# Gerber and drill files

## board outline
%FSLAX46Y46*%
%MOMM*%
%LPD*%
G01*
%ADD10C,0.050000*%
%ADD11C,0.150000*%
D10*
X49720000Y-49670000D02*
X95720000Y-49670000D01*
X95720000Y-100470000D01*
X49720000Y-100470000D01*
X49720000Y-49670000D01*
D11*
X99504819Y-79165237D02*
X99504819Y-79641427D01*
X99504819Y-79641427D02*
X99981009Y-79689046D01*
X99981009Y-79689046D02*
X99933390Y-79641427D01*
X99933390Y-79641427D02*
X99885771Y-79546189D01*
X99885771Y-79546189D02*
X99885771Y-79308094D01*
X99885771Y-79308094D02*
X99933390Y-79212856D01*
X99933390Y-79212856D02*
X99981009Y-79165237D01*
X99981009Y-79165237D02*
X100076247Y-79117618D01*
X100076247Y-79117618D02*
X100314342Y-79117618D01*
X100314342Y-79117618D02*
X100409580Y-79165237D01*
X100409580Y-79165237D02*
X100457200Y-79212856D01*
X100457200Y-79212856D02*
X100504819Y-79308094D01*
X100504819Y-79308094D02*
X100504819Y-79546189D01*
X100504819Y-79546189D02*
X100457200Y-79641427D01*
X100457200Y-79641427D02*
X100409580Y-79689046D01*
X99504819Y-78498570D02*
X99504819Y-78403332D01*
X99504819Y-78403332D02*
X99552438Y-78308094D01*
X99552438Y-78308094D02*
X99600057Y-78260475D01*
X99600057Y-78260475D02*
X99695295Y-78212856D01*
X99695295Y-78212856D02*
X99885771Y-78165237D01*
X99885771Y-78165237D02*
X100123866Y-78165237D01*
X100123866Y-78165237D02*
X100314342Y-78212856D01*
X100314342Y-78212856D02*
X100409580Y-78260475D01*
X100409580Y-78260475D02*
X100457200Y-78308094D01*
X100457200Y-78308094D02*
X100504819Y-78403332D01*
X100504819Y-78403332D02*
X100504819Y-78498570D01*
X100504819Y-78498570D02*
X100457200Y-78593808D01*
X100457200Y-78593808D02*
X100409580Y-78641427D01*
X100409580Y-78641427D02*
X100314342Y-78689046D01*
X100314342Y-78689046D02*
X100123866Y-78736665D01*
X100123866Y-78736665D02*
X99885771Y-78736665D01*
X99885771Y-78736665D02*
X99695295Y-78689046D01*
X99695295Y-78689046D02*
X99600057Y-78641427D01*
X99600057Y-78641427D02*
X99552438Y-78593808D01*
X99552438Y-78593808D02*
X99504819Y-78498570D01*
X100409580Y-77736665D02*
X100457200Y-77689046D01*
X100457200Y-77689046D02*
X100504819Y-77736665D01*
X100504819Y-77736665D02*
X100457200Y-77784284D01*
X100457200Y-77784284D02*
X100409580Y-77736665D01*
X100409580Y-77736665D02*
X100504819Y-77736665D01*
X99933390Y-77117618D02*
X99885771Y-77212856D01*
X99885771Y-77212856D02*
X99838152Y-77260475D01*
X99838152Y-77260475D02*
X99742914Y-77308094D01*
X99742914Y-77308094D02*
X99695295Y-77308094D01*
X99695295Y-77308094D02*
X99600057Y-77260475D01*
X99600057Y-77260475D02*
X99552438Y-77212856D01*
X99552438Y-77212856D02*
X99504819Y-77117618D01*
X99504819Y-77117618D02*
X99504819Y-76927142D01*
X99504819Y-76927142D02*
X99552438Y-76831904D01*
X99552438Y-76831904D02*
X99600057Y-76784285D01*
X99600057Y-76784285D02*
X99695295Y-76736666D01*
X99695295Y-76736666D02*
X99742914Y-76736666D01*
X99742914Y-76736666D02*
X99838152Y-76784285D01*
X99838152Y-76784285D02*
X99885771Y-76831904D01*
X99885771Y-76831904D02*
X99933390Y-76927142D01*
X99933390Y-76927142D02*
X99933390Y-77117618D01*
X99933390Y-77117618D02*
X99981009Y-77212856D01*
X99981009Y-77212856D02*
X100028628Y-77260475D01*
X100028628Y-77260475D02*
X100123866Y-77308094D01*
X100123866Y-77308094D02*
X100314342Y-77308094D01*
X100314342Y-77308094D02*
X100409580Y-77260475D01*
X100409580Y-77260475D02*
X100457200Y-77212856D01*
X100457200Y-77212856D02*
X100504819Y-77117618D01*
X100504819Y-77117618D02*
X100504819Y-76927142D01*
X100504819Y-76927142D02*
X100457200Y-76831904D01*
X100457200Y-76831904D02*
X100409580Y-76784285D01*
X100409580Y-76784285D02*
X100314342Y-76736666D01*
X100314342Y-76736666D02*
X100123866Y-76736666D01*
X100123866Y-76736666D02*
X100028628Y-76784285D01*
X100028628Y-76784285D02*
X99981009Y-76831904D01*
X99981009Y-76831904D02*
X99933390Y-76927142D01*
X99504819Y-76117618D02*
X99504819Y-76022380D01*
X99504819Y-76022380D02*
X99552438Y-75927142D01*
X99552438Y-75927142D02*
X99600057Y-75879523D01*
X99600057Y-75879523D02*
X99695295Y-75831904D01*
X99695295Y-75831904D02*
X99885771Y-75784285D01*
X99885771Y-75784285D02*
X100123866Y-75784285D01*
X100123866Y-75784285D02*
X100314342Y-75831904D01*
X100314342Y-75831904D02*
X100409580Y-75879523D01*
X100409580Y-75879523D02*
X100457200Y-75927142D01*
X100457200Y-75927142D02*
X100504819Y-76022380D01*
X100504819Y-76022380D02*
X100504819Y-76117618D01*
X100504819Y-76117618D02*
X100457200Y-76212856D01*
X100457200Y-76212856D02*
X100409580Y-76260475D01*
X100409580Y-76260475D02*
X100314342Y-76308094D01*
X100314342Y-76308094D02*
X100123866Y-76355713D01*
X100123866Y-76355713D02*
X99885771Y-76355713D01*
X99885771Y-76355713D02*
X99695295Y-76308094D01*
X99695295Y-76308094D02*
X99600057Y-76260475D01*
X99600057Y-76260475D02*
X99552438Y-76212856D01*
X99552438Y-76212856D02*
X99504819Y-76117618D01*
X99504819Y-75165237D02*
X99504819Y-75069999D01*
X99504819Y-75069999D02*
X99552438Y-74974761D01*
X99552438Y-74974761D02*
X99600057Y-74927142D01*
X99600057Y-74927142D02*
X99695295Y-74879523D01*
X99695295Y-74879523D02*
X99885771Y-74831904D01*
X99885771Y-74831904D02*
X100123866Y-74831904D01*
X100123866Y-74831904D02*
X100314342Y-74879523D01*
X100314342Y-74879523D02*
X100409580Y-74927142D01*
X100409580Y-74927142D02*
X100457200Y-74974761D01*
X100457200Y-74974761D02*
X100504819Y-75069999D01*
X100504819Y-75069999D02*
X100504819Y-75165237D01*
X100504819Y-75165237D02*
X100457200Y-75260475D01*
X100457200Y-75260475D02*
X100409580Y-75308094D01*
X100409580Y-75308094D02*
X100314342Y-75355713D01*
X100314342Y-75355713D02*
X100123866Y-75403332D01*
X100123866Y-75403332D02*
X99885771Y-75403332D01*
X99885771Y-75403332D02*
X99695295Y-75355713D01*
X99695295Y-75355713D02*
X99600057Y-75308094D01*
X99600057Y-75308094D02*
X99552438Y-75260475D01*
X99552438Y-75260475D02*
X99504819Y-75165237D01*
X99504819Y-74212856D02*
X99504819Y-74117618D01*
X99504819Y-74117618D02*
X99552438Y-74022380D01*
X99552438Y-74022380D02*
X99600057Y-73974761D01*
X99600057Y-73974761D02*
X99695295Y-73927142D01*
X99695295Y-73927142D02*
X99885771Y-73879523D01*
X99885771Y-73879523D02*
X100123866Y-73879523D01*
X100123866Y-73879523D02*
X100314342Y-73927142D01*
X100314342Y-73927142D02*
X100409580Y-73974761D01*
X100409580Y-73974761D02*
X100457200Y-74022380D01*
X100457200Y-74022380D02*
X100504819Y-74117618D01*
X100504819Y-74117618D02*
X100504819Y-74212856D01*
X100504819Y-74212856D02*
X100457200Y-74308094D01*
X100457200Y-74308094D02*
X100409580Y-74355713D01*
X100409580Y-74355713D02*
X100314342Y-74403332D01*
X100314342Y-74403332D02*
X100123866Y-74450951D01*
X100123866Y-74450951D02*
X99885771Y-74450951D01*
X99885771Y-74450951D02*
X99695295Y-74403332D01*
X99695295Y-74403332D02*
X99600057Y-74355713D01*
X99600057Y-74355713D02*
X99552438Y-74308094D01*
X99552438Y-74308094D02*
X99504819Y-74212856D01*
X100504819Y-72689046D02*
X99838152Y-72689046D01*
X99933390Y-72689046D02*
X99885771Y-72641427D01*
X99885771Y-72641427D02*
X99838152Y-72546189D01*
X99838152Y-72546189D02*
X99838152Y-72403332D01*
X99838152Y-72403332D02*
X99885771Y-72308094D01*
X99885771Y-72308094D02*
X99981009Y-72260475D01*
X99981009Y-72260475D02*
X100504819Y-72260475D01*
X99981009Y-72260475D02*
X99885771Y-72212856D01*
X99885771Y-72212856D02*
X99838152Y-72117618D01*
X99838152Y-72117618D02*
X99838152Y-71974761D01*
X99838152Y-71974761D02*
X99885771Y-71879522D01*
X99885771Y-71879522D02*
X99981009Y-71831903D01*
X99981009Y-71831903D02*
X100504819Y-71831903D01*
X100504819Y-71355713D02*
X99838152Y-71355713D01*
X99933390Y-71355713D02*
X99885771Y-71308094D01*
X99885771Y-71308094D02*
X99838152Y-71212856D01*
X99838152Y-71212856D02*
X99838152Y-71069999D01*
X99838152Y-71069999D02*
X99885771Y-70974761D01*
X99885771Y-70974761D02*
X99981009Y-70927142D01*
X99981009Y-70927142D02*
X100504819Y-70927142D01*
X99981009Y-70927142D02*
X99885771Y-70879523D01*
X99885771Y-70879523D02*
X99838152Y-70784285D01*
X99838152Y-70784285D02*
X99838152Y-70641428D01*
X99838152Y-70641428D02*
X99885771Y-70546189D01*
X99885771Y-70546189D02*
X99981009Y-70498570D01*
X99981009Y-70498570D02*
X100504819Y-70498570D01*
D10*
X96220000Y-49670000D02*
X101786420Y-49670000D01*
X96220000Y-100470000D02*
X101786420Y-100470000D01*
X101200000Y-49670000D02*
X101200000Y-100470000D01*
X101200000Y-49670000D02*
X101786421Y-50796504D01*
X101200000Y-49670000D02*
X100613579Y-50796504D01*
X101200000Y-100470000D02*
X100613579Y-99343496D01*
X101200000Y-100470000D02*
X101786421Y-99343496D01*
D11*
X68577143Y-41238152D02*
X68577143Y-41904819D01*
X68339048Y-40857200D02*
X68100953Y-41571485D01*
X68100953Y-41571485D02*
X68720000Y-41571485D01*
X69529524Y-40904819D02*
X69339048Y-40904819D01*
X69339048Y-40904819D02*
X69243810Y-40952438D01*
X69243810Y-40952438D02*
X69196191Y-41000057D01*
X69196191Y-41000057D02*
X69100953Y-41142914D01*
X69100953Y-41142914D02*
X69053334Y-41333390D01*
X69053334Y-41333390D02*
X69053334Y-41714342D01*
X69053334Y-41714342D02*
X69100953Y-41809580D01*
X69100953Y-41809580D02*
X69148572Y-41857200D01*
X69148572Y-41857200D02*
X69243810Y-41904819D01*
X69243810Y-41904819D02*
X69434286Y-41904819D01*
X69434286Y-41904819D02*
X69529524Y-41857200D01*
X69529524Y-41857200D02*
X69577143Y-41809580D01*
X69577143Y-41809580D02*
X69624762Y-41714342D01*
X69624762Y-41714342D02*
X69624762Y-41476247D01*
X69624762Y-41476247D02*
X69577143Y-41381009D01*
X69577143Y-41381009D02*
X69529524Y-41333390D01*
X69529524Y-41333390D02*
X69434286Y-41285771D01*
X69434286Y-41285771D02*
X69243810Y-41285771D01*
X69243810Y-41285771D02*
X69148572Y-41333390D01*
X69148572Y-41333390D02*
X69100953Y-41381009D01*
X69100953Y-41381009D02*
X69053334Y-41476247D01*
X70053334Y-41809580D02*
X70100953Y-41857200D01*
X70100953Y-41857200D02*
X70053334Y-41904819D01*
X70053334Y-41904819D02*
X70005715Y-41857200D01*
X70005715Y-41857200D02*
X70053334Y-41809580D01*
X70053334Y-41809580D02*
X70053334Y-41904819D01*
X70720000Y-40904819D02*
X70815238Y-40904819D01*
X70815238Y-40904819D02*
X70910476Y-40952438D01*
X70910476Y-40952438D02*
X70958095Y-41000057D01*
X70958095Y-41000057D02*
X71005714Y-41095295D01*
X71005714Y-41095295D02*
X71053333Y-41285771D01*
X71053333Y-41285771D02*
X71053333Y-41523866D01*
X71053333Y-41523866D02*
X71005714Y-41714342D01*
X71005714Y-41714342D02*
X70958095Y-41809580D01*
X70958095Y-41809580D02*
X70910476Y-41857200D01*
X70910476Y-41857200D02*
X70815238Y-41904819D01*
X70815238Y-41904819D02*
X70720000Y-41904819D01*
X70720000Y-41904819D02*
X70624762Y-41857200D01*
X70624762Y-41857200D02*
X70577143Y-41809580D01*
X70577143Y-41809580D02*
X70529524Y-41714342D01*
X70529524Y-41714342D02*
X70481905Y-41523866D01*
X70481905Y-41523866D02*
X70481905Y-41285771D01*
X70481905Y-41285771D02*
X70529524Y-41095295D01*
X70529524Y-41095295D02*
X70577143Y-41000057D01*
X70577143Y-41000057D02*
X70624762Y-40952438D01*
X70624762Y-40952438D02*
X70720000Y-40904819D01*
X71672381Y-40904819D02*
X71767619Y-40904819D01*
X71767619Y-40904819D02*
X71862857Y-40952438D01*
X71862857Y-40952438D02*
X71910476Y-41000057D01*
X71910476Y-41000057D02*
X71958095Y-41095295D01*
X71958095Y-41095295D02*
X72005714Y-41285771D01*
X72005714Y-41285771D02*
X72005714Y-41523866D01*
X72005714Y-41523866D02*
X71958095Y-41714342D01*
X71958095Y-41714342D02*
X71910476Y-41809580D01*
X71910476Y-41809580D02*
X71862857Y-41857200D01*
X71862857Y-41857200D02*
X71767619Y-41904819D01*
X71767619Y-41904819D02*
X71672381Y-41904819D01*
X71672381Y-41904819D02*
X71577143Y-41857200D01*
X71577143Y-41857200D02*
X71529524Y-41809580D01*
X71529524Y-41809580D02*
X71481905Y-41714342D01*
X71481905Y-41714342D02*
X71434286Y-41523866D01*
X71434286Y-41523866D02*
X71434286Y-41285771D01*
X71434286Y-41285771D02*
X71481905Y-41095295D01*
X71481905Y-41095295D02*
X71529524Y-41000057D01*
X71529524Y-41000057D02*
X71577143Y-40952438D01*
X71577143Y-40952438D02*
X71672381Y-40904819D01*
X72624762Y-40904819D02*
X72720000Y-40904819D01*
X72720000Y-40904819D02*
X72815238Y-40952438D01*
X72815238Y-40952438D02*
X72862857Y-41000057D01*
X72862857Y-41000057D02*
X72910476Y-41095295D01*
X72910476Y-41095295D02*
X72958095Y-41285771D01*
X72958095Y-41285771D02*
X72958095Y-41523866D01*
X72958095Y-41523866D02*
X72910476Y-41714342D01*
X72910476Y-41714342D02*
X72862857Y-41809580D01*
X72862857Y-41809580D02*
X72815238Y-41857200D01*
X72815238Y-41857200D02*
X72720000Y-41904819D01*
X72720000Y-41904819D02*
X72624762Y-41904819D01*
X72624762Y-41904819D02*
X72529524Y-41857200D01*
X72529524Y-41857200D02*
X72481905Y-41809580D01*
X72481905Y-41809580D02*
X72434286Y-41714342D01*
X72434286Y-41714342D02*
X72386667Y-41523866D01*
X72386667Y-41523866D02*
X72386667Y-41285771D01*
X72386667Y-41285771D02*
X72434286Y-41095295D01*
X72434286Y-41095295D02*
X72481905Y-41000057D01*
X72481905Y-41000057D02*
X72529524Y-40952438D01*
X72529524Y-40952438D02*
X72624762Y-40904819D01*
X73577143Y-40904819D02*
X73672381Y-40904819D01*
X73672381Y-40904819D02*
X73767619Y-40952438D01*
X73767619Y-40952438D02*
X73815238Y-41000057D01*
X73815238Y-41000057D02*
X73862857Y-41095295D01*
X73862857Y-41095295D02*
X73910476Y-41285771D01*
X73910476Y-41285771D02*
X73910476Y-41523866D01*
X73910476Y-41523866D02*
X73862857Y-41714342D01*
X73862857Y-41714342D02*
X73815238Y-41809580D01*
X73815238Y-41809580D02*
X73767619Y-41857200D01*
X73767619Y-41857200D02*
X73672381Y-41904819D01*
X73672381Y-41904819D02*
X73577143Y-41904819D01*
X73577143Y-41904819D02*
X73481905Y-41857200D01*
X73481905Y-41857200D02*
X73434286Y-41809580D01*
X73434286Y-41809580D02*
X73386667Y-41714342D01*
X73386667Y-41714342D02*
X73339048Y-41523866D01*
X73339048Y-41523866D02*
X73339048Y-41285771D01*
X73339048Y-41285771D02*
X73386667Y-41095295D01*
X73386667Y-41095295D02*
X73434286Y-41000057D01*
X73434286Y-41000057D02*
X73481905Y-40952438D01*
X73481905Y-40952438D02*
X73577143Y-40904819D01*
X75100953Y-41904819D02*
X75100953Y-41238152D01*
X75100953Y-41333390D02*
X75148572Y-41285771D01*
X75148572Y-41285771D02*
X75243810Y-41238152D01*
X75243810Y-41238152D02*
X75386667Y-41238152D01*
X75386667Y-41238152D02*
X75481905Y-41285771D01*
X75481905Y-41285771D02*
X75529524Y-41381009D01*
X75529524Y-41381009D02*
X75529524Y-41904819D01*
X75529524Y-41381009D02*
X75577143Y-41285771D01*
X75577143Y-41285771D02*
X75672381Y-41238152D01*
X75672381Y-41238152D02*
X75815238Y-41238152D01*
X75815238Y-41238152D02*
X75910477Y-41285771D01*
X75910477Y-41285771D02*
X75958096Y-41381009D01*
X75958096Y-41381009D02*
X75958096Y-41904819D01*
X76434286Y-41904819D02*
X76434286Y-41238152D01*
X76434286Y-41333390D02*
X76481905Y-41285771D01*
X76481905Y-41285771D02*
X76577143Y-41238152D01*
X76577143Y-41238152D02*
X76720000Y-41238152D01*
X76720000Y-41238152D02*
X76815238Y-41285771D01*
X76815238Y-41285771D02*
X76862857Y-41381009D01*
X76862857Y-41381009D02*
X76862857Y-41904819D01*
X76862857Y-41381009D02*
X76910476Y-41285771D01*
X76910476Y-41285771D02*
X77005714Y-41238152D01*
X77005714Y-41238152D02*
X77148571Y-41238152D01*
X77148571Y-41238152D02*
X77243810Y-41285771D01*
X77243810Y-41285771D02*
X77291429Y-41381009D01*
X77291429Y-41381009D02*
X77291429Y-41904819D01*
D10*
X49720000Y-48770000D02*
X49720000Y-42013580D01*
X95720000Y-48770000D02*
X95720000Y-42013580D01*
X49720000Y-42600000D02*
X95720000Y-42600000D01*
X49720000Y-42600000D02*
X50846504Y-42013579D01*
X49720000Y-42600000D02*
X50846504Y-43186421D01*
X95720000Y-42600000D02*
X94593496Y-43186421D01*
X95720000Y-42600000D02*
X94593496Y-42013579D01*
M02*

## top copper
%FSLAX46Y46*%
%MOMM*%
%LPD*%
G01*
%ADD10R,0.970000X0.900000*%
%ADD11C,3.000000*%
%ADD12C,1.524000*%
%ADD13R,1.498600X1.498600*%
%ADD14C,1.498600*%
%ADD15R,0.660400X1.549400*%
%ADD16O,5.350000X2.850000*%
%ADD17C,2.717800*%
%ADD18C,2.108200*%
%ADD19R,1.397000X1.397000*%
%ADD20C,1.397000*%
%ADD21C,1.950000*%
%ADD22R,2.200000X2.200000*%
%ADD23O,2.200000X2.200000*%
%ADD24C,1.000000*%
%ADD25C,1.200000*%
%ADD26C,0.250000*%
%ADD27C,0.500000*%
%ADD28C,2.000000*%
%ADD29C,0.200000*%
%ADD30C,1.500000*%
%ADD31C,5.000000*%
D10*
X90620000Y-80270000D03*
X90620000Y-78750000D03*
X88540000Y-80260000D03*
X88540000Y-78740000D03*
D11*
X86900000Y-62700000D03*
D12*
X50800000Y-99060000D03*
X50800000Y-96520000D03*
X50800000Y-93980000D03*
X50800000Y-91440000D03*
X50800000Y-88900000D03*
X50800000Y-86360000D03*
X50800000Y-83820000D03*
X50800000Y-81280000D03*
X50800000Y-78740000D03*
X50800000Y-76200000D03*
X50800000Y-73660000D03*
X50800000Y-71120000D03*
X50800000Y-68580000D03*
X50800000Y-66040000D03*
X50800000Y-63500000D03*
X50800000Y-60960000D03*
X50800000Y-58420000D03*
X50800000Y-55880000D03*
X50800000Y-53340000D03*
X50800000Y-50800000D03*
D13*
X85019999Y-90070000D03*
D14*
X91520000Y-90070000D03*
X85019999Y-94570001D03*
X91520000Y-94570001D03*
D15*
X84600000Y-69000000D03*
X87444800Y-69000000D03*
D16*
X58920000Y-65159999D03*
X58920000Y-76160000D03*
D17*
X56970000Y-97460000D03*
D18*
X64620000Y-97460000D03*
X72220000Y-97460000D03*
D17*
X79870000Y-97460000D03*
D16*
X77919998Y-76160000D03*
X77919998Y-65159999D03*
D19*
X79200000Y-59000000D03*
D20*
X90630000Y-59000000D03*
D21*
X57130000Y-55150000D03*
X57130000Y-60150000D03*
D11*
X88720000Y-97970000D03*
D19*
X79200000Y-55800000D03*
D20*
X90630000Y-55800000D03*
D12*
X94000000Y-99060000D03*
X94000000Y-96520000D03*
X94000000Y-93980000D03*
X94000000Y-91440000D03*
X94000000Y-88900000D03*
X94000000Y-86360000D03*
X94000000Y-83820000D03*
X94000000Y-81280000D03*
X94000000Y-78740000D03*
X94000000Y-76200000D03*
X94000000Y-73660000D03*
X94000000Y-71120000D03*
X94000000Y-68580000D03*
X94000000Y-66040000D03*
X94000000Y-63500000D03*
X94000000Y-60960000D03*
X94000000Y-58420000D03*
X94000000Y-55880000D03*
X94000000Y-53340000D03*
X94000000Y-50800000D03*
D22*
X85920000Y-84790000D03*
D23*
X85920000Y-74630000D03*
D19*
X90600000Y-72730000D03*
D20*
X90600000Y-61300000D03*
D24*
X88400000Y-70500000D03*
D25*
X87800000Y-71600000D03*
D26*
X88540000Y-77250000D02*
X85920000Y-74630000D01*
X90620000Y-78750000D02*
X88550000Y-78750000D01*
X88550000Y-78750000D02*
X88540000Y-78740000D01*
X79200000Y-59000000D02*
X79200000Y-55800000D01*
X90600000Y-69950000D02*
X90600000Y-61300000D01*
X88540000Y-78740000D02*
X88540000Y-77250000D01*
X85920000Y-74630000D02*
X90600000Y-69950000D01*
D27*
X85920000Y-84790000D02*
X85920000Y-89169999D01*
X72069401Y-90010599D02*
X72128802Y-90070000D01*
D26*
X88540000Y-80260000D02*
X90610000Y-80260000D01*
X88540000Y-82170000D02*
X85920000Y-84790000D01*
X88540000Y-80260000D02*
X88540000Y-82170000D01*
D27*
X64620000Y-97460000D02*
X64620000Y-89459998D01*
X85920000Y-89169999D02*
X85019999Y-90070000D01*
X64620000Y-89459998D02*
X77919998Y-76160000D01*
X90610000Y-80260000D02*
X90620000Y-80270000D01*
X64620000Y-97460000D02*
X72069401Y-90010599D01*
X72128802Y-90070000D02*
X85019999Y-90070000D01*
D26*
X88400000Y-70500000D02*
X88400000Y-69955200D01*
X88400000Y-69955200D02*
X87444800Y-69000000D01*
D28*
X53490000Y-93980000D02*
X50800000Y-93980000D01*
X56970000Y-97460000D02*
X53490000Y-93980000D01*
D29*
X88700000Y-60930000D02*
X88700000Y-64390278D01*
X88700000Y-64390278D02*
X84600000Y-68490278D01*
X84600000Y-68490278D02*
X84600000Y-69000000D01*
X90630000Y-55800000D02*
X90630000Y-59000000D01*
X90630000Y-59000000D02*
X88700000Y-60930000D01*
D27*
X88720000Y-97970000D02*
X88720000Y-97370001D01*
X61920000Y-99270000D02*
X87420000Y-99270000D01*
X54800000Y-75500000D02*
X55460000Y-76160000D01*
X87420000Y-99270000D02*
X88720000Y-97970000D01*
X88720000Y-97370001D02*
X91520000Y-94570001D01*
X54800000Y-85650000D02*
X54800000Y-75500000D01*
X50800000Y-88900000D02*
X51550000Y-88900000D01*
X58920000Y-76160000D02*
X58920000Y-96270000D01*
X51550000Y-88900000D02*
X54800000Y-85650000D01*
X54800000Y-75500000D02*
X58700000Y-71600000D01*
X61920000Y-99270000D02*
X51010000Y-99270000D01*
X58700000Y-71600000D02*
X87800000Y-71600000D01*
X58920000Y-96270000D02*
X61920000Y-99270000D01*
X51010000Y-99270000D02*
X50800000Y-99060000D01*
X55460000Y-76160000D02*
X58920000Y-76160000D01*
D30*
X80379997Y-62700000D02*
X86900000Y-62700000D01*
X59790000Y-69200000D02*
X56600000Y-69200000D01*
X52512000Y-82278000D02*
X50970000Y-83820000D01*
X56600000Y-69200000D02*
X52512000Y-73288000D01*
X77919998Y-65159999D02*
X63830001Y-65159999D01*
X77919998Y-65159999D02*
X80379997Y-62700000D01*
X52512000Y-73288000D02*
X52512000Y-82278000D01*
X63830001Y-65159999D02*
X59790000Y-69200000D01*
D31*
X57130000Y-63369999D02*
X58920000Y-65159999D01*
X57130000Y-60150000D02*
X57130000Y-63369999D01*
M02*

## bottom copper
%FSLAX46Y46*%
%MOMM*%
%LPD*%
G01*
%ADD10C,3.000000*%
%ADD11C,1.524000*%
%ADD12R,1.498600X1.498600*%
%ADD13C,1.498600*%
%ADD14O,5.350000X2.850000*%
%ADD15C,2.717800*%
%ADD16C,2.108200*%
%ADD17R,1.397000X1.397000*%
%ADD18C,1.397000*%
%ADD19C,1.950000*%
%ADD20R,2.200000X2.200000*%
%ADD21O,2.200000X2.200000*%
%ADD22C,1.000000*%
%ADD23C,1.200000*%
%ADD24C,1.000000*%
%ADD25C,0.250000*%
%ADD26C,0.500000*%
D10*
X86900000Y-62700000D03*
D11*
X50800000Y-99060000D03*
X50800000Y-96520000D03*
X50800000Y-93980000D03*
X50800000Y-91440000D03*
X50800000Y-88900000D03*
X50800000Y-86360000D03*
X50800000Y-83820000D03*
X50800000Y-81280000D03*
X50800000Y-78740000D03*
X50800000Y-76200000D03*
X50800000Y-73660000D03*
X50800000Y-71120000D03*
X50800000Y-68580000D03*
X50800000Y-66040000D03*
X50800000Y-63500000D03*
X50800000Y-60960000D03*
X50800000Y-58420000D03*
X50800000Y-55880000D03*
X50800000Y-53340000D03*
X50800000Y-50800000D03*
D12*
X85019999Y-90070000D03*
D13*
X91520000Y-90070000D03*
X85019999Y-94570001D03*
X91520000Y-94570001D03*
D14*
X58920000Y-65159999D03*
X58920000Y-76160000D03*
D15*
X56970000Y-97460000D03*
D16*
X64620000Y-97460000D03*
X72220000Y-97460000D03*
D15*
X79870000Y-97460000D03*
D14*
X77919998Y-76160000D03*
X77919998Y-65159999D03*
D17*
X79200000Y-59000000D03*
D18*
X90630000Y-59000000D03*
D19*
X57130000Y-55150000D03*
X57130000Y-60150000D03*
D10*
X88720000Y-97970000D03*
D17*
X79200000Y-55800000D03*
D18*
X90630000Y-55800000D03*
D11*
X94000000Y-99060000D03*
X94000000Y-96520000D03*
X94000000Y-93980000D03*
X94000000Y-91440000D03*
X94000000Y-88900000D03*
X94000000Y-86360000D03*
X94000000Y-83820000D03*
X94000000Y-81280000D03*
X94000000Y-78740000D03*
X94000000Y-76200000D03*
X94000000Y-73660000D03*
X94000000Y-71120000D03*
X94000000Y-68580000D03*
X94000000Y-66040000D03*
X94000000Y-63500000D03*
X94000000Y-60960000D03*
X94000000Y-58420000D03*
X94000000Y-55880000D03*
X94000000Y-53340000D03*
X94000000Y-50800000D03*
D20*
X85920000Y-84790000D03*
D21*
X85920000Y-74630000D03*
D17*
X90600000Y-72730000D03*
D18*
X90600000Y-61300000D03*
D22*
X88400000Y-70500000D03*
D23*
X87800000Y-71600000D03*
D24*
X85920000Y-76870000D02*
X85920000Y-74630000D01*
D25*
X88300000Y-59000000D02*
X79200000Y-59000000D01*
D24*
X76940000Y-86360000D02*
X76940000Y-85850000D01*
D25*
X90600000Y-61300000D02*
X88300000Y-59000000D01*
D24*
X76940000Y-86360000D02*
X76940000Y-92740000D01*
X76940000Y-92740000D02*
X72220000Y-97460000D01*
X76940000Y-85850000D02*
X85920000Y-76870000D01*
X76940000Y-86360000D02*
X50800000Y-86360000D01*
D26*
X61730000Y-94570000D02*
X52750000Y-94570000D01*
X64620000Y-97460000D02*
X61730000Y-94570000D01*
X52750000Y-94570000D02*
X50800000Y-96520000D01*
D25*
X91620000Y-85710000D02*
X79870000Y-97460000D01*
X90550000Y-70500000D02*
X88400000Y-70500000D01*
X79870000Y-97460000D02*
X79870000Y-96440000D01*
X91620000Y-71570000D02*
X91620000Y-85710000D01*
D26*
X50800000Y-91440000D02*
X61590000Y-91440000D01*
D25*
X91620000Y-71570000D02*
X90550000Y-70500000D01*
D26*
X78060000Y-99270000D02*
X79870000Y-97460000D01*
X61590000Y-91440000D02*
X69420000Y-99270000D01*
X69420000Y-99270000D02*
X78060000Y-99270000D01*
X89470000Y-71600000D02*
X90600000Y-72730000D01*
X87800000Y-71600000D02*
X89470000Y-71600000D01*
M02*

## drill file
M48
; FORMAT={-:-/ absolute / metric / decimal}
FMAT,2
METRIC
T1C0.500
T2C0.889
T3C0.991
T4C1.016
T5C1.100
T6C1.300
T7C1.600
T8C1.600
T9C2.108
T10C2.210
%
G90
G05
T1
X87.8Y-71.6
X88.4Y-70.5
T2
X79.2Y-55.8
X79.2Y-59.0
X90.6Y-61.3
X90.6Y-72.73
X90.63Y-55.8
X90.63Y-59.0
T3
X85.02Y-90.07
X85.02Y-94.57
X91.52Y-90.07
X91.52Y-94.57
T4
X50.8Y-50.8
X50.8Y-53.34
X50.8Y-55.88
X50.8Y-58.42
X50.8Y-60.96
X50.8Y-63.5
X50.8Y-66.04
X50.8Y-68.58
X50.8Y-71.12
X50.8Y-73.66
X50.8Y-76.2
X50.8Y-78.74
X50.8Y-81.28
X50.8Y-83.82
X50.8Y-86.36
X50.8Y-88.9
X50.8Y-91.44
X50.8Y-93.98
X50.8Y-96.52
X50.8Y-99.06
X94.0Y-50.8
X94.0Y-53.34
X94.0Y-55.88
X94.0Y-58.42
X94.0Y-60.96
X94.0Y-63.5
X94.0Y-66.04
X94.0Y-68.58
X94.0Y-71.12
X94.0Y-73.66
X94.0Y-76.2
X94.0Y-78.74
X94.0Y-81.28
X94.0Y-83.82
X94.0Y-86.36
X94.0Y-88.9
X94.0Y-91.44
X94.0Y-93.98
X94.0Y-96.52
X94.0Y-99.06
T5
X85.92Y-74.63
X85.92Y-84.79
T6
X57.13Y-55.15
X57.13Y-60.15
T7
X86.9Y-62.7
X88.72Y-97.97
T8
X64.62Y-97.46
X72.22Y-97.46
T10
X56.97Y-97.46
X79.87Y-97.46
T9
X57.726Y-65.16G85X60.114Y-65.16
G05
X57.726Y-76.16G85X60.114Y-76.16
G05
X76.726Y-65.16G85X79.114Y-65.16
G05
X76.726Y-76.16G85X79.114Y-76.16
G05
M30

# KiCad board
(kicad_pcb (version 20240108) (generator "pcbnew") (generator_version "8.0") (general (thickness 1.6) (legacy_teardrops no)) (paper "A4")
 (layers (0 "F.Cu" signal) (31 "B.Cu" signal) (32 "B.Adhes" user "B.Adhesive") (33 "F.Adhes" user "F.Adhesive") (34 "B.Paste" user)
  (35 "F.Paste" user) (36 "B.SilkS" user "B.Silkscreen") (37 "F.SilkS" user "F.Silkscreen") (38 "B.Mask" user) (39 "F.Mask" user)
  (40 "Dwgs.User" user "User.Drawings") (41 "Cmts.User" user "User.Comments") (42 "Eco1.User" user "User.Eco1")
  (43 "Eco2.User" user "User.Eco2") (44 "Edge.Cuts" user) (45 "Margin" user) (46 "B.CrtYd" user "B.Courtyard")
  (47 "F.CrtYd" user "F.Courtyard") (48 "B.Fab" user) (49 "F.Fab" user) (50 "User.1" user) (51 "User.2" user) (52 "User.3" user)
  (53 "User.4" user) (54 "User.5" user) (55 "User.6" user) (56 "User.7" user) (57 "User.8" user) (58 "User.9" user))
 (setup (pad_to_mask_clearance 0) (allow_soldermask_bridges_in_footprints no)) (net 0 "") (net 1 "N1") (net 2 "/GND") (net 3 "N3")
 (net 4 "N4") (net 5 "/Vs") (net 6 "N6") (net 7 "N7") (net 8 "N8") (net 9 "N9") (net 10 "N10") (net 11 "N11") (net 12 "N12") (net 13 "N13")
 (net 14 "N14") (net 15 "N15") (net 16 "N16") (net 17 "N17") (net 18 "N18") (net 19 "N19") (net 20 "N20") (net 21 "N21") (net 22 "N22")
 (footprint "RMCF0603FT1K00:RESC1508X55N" (layer "F.Cu") (at 90.62 79.51 90)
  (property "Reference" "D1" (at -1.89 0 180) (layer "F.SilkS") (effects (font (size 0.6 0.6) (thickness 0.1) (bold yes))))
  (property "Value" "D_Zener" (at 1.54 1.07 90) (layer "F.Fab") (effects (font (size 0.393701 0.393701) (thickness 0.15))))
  (pad "1" smd rect (at -0.76 0 90) (size 0.9 0.97) (layers "F.Cu" "F.Paste" "F.Mask") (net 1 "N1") (solder_mask_margin 0.102))
  (pad "2" smd rect (at 0.76 0 90) (size 0.9 0.97) (layers "F.Cu" "F.Paste" "F.Mask") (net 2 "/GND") (solder_mask_margin 0.102)))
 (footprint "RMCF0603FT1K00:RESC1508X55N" (layer "F.Cu") (at 88.54 79.5 90)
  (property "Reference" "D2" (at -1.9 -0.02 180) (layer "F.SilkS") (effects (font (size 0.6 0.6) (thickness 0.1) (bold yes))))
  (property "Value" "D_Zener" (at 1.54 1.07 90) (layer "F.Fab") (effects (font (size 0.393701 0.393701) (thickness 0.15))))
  (pad "1" smd rect (at -0.76 0 90) (size 0.9 0.97) (layers "F.Cu" "F.Paste" "F.Mask") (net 1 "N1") (solder_mask_margin 0.102))
  (pad "2" smd rect (at 0.76 0 90) (size 0.9 0.97) (layers "F.Cu" "F.Paste" "F.Mask") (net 2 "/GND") (solder_mask_margin 0.102)))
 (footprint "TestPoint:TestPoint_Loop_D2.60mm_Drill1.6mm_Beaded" (layer "F.Cu") (at 86.9 62.7)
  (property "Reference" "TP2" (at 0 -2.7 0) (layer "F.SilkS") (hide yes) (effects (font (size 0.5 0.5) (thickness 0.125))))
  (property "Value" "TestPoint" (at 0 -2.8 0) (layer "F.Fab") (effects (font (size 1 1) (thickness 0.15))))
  (pad "1" thru_hole circle (at 0 0) (size 3 3) (drill 1.6) (layers "*.Cu" "*.Mask") (remove_unused_layers no) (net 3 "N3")))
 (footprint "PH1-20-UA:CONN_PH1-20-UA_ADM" (layer "F.Cu") (at 50.8 99.06 90)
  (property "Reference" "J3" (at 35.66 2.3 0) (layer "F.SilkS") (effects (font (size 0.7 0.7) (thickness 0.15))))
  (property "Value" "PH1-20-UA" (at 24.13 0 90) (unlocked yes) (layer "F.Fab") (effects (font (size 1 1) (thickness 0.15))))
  (pad "1" thru_hole circle (at 0 0 90) (size 1.524 1.524) (drill 1.016) (layers "*.Cu" "*.Mask") (remove_unused_layers no) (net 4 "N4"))
  (pad "2" thru_hole circle (at 2.54 0 90) (size 1.524 1.524) (drill 1.016) (layers "*.Cu" "*.Mask") (remove_unused_layers no) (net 1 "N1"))
  (pad "3" thru_hole circle (at 5.08 0 90) (size 1.524 1.524) (drill 1.016) (layers "*.Cu" "*.Mask") (remove_unused_layers no) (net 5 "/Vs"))
  (pad "4" thru_hole circle (at 7.62 0 90) (size 1.524 1.524) (drill 1.016) (layers "*.Cu" "*.Mask") (remove_unused_layers no) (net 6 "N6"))
  (pad "5" thru_hole circle (at 10.16 0 90) (size 1.524 1.524) (drill 1.016) (layers "*.Cu" "*.Mask") (remove_unused_layers no) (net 4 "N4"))
  (pad "6" thru_hole circle (at 12.7 0 90) (size 1.524 1.524) (drill 1.016) (layers "*.Cu" "*.Mask") (remove_unused_layers no)
   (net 2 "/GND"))
  (pad "7" thru_hole circle (at 15.24 0 90) (size 1.524 1.524) (drill 1.016) (layers "*.Cu" "*.Mask") (remove_unused_layers no) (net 3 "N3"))
  (pad "8" thru_hole circle (at 17.78 0 90) (size 1.524 1.524) (drill 1.016) (layers "*.Cu" "*.Mask") (remove_unused_layers no) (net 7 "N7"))
  (pad "9" thru_hole circle (at 20.32 0 90) (size 1.524 1.524) (drill 1.016) (layers "*.Cu" "*.Mask") (remove_unused_layers no) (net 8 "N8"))
  (pad "10" thru_hole circle (at 22.86 0 90) (size 1.524 1.524) (drill 1.016) (layers "*.Cu" "*.Mask") (remove_unused_layers no)
   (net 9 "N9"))
  (pad "11" thru_hole circle (at 25.4 0 90) (size 1.524 1.524) (drill 1.016) (layers "*.Cu" "*.Mask") (remove_unused_layers no)
   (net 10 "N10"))
  (pad "12" thru_hole circle (at 27.94 0 90) (size 1.524 1.524) (drill 1.016) (layers "*.Cu" "*.Mask") (remove_unused_layers no)
   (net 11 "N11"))
  (pad "13" thru_hole circle (at 30.48 0 90) (size 1.524 1.524) (drill 1.016) (layers "*.Cu" "*.Mask") (remove_unused_layers no)
   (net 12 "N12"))
  (pad "14" thru_hole circle (at 33.02 0 90) (size 1.524 1.524) (drill 1.016) (layers "*.Cu" "*.Mask") (remove_unused_layers no)
   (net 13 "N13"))
  (pad "15" thru_hole circle (at 35.56 0 90) (size 1.524 1.524) (drill 1.016) (layers "*.Cu" "*.Mask") (remove_unused_layers no)
   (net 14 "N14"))
  (pad "16" thru_hole circle (at 38.1 0 90) (size 1.524 1.524) (drill 1.016) (layers "*.Cu" "*.Mask") (remove_unused_layers no)
   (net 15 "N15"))
  (pad "17" thru_hole circle (at 40.64 0 90) (size 1.524 1.524) (drill 1.016) (layers "*.Cu" "*.Mask") (remove_unused_layers no)
   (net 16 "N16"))
  (pad "18" thru_hole circle (at 43.18 0 90) (size 1.524 1.524) (drill 1.016) (layers "*.Cu" "*.Mask") (remove_unused_layers no)
   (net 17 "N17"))
  (pad "19" thru_hole circle (at 45.72 0 90) (size 1.524 1.524) (drill 1.016) (layers "*.Cu" "*.Mask") (remove_unused_layers no)
   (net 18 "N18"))
  (pad "20" thru_hole circle (at 48.26 0 90) (size 1.524 1.524) (drill 1.016) (layers "*.Cu" "*.Mask") (remove_unused_layers no)
   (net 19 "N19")))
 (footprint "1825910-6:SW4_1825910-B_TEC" (layer "F.Cu") (at 91.52 94.570001)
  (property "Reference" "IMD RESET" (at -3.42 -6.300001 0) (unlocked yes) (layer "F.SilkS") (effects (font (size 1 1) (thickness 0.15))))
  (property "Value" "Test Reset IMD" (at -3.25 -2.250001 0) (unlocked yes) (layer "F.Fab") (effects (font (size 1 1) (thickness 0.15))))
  (pad "1" thru_hole rect (at -6.500001 -4.500001) (size 1.4986 1.4986) (drill 0.9906) (layers "*.Cu" "*.Mask") (remove_unused_layers no)
   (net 1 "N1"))
  (pad "2" thru_hole circle (at 0 -4.500001) (size 1.4986 1.4986) (drill 0.9906) (layers "*.Cu" "*.Mask") (remove_unused_layers no))
  (pad "3" thru_hole circle (at -6.500001 0) (size 1.4986 1.4986) (drill 0.9906) (layers "*.Cu" "*.Mask") (remove_unused_layers no))
  (pad "4" thru_hole circle (at 0 0) (size 1.4986 1.4986) (drill 0.9906) (layers "*.Cu" "*.Mask") (remove_unused_layers no) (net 4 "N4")))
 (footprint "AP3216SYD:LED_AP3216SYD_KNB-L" (layer "F.Cu") (at 86.0224 69)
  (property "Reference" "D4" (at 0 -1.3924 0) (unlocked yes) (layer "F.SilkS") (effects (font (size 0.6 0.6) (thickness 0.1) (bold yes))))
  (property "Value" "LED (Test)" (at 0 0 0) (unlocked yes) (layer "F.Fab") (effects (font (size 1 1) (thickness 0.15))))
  (pad "1" smd rect (at -1.4224 0) (size 0.6604 1.5494) (layers "F.Cu" "F.Paste" "F.Mask") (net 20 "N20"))
  (pad "2" smd rect (at 1.4224 0) (size 0.6604 1.5494) (layers "F.Cu" "F.Paste" "F.Mask") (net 6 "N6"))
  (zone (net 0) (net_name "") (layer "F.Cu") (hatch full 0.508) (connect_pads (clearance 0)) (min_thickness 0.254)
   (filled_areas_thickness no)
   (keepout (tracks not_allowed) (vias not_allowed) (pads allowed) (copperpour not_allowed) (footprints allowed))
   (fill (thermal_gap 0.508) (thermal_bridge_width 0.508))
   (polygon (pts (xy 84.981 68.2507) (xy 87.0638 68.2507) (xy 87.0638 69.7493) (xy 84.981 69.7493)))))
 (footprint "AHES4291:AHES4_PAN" (layer "F.Cu") (at 58.919999 65.159998)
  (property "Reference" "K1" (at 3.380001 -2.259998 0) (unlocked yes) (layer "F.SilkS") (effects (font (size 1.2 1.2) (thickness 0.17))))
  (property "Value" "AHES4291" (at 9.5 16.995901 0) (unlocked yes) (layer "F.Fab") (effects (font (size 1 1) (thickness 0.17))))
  (pad "1" thru_hole oval (at 0.000001 0.000001) (size 5.35 2.85) (drill oval 4.4958 2.1082) (layers "*.Cu" "*.Mask")
   (remove_unused_layers no) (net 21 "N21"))
  (pad "2" thru_hole oval (at 0.000001 11.000002) (size 5.35 2.85) (drill oval 4.4958 2.1082) (layers "*.Cu" "*.Mask")
   (remove_unused_layers no) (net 4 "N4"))
  (pad "3" thru_hole circle (at -1.949999 32.300002) (size 2.7178 2.7178) (drill 2.2098) (layers "*.Cu" "*.Mask") (remove_unused_layers no)
   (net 5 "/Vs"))
  (pad "4" thru_hole circle (at 5.700001 32.300002) (size 2.1082 2.1082) (drill 1.6002) (layers "*.Cu" "*.Mask") (remove_unused_layers no)
   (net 1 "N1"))
  (pad "5" thru_hole circle (at 13.300001 32.300002) (size 2.1082 2.1082) (drill 1.6002) (layers "*.Cu" "*.Mask") (remove_unused_layers no)
   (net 2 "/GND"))
  (pad "6" thru_hole circle (at 20.950001 32.300002) (size 2.7178 2.7178) (drill 2.2098) (layers "*.Cu" "*.Mask") (remove_unused_layers no)
   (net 6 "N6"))
  (pad "7" thru_hole oval (at 18.999999 11.000002) (size 5.35 2.85) (drill oval 4.4958 2.1082) (layers "*.Cu" "*.Mask")
   (remove_unused_layers no) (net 1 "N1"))
  (pad "8" thru_hole oval (at 18.999999 0.000001) (size 5.35 2.85) (drill oval 4.4958 2.1082) (layers "*.Cu" "*.Mask")
   (remove_unused_layers no) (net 3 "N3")))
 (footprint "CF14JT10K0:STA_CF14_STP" (layer "F.Cu") (at 79.2 59)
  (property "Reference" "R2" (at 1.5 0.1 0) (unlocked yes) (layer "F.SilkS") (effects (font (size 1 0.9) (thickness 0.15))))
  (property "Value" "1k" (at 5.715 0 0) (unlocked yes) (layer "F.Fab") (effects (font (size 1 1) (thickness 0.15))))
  (pad "1" thru_hole rect (at 0 0) (size 1.397 1.397) (drill 0.889) (layers "*.Cu" "*.Mask") (remove_unused_layers no) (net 2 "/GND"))
  (pad "2" thru_hole circle (at 11.43 0) (size 1.397 1.397) (drill 0.889) (layers "*.Cu" "*.Mask") (remove_unused_layers no) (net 20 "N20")))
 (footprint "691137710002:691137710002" (layer "F.Cu") (at 57.13 57.65 -90)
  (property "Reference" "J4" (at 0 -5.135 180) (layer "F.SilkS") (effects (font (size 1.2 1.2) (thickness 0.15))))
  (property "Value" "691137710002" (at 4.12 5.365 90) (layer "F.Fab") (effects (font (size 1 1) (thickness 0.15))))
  (pad "1" thru_hole circle (at -2.5 0 270) (size 1.95 1.95) (drill 1.3) (layers "*.Cu" "*.Mask") (remove_unused_layers no) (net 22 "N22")
   (solder_mask_margin 0.102))
  (pad "2" thru_hole circle (at 2.5 0 270) (size 1.95 1.95) (drill 1.3) (layers "*.Cu" "*.Mask") (remove_unused_layers no) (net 21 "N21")
   (solder_mask_margin 0.102)))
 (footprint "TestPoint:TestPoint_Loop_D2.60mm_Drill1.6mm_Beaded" (layer "F.Cu") (at 88.72 97.97)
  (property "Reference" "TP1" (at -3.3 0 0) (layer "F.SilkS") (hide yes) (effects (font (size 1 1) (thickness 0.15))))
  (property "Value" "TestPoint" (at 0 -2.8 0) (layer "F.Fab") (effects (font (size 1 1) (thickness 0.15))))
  (pad "1" thru_hole circle (at 0 0) (size 3 3) (drill 1.6) (layers "*.Cu" "*.Mask") (remove_unused_layers no) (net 4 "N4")))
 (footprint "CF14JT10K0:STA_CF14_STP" (layer "F.Cu") (at 79.2 55.8)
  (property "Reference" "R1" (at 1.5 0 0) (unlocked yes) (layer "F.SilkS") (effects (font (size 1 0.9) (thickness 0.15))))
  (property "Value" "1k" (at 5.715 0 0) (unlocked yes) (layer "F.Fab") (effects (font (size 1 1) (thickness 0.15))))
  (pad "1" thru_hole rect (at 0 0) (size 1.397 1.397) (drill 0.889) (layers "*.Cu" "*.Mask") (remove_unused_layers no) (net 2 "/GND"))
  (pad "2" thru_hole circle (at 11.43 0) (size 1.397 1.397) (drill 0.889) (layers "*.Cu" "*.Mask") (remove_unused_layers no) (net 20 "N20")))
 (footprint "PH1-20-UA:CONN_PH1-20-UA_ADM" (layer "F.Cu") (at 94 99.06 90)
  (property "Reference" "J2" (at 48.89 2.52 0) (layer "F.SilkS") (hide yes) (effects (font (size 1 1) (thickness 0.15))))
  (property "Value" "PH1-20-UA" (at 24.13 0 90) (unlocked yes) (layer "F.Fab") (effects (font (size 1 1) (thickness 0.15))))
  (pad "1" thru_hole circle (at 0 0 90) (size 1.524 1.524) (drill 1.016) (layers "*.Cu" "*.Mask") (remove_unused_layers no))
  (pad "2" thru_hole circle (at 2.54 0 90) (size 1.524 1.524) (drill 1.016) (layers "*.Cu" "*.Mask") (remove_unused_layers no))
  (pad "3" thru_hole circle (at 5.08 0 90) (size 1.524 1.524) (drill 1.016) (layers "*.Cu" "*.Mask") (remove_unused_layers no))
  (pad "4" thru_hole circle (at 7.62 0 90) (size 1.524 1.524) (drill 1.016) (layers "*.Cu" "*.Mask") (remove_unused_layers no))
  (pad "5" thru_hole circle (at 10.16 0 90) (size 1.524 1.524) (drill 1.016) (layers "*.Cu" "*.Mask") (remove_unused_layers no))
  (pad "6" thru_hole circle (at 12.7 0 90) (size 1.524 1.524) (drill 1.016) (layers "*.Cu" "*.Mask") (remove_unused_layers no))
  (pad "7" thru_hole circle (at 15.24 0 90) (size 1.524 1.524) (drill 1.016) (layers "*.Cu" "*.Mask") (remove_unused_layers no))
  (pad "8" thru_hole circle (at 17.78 0 90) (size 1.524 1.524) (drill 1.016) (layers "*.Cu" "*.Mask") (remove_unused_layers no))
  (pad "9" thru_hole circle (at 20.32 0 90) (size 1.524 1.524) (drill 1.016) (layers "*.Cu" "*.Mask") (remove_unused_layers no))
  (pad "10" thru_hole circle (at 22.86 0 90) (size 1.524 1.524) (drill 1.016) (layers "*.Cu" "*.Mask") (remove_unused_layers no))
  (pad "11" thru_hole circle (at 25.4 0 90) (size 1.524 1.524) (drill 1.016) (layers "*.Cu" "*.Mask") (remove_unused_layers no))
  (pad "12" thru_hole circle (at 27.94 0 90) (size 1.524 1.524) (drill 1.016) (layers "*.Cu" "*.Mask") (remove_unused_layers no))
  (pad "13" thru_hole circle (at 30.48 0 90) (size 1.524 1.524) (drill 1.016) (layers "*.Cu" "*.Mask") (remove_unused_layers no))
  (pad "14" thru_hole circle (at 33.02 0 90) (size 1.524 1.524) (drill 1.016) (layers "*.Cu" "*.Mask") (remove_unused_layers no))
  (pad "15" thru_hole circle (at 35.56 0 90) (size 1.524 1.524) (drill 1.016) (layers "*.Cu" "*.Mask") (remove_unused_layers no))
  (pad "16" thru_hole circle (at 38.1 0 90) (size 1.524 1.524) (drill 1.016) (layers "*.Cu" "*.Mask") (remove_unused_layers no))
  (pad "17" thru_hole circle (at 40.64 0 90) (size 1.524 1.524) (drill 1.016) (layers "*.Cu" "*.Mask") (remove_unused_layers no))
  (pad "18" thru_hole circle (at 43.18 0 90) (size 1.524 1.524) (drill 1.016) (layers "*.Cu" "*.Mask") (remove_unused_layers no))
  (pad "19" thru_hole circle (at 45.72 0 90) (size 1.524 1.524) (drill 1.016) (layers "*.Cu" "*.Mask") (remove_unused_layers no))
  (pad "20" thru_hole circle (at 48.26 0 90) (size 1.524 1.524) (drill 1.016) (layers "*.Cu" "*.Mask") (remove_unused_layers no)))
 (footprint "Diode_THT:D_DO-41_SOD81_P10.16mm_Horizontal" (layer "F.Cu") (at 85.92 84.79 90)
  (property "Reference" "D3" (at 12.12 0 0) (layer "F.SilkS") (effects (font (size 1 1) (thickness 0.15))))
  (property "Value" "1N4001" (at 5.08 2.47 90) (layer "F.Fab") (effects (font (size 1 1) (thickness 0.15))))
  (pad "1" thru_hole rect (at 0 0 90) (size 2.2 2.2) (drill 1.1) (layers "*.Cu" "*.Mask") (remove_unused_layers no) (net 1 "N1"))
  (pad "2" thru_hole oval (at 10.16 0 90) (size 2.2 2.2) (drill 1.1) (layers "*.Cu" "*.Mask") (remove_unused_layers no) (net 2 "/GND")))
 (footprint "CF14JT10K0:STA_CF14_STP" (layer "F.Cu") (at 90.6 72.73 90)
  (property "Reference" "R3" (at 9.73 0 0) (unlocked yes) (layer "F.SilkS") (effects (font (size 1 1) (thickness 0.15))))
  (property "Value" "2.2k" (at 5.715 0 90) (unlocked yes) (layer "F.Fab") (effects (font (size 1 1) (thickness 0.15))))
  (pad "1" thru_hole rect (at 0 0 90) (size 1.397 1.397) (drill 0.889) (layers "*.Cu" "*.Mask") (remove_unused_layers no) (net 4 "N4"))
  (pad "2" thru_hole circle (at 11.43 0 90) (size 1.397 1.397) (drill 0.889) (layers "*.Cu" "*.Mask") (remove_unused_layers no)
   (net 2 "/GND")))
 (gr_rect (start 49.72 49.67) (end 95.72 100.47) (stroke (width 0.05) (type default)) (fill none) (layer "Edge.Cuts"))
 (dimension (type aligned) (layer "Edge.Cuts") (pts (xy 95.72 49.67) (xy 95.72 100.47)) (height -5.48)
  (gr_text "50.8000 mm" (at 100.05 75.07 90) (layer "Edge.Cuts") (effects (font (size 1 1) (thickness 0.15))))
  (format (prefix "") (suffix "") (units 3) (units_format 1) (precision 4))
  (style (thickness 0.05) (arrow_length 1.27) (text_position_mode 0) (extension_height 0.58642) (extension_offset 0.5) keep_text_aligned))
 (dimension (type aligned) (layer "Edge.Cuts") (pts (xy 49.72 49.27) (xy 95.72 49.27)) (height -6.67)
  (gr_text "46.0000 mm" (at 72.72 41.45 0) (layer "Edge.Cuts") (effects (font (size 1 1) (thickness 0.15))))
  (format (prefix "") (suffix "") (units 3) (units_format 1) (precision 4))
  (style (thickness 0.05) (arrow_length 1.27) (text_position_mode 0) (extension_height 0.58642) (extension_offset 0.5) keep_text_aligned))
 (segment (start 88.54 77.25) (end 85.92 74.63) (width 0.25) (layer "F.Cu") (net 2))
 (segment (start 90.62 78.75) (end 88.55 78.75) (width 0.25) (layer "F.Cu") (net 2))
 (segment (start 88.55 78.75) (end 88.54 78.74) (width 0.25) (layer "F.Cu") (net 2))
 (segment (start 79.2 59) (end 79.2 55.8) (width 0.25) (layer "F.Cu") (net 2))
 (segment (start 90.6 69.95) (end 90.6 61.3) (width 0.25) (layer "F.Cu") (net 2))
 (segment (start 88.54 78.74) (end 88.54 77.25) (width 0.25) (layer "F.Cu") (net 2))
 (segment (start 85.92 74.63) (end 90.6 69.95) (width 0.25) (layer "F.Cu") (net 2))
 (segment (start 85.92 76.87) (end 85.92 74.63) (width 1) (layer "B.Cu") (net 2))
 (segment (start 88.3 59) (end 79.2 59) (width 0.25) (layer "B.Cu") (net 2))
 (segment (start 76.94 86.36) (end 76.94 85.85) (width 1) (layer "B.Cu") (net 2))
 (segment (start 90.6 61.3) (end 88.3 59) (width 0.25) (layer "B.Cu") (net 2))
 (segment (start 76.94 86.36) (end 76.94 92.74) (width 1) (layer "B.Cu") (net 2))
 (segment (start 76.94 92.74) (end 72.22 97.46) (width 1) (layer "B.Cu") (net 2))
 (segment (start 76.94 85.85) (end 85.92 76.87) (width 1) (layer "B.Cu") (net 2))
 (segment (start 76.94 86.36) (end 50.8 86.36) (width 1) (layer "B.Cu") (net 2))
 (segment (start 85.92 84.79) (end 85.92 89.169999) (width 0.5) (layer "F.Cu") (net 1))
 (segment (start 72.069401 90.010599) (end 72.128802 90.07) (width 0.5) (layer "F.Cu") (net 1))
 (segment (start 88.54 80.26) (end 90.61 80.26) (width 0.25) (layer "F.Cu") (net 1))
 (segment (start 88.54 82.17) (end 85.92 84.79) (width 0.25) (layer "F.Cu") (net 1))
 (segment (start 88.54 80.26) (end 88.54 82.17) (width 0.25) (layer "F.Cu") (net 1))
 (segment (start 64.62 97.46) (end 64.62 89.459998) (width 0.5) (layer "F.Cu") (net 1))
 (segment (start 85.92 89.169999) (end 85.019999 90.07) (width 0.5) (layer "F.Cu") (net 1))
 (segment (start 64.62 89.459998) (end 77.919998 76.16) (width 0.5) (layer "F.Cu") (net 1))
 (segment (start 90.61 80.26) (end 90.62 80.27) (width 0.5) (layer "F.Cu") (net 1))
 (segment (start 64.62 97.46) (end 72.069401 90.010599) (width 0.5) (layer "F.Cu") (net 1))
 (segment (start 72.128802 90.07) (end 85.019999 90.07) (width 0.5) (layer "F.Cu") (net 1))
 (segment (start 61.73 94.57) (end 52.75 94.57) (width 0.5) (layer "B.Cu") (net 1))
 (segment (start 64.62 97.46) (end 61.73 94.57) (width 0.5) (layer "B.Cu") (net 1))
 (segment (start 52.75 94.57) (end 50.8 96.52) (width 0.5) (layer "B.Cu") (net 1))
 (segment (start 88.4 70.5) (end 88.4 69.9552) (width 0.25) (layer "F.Cu") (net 6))
 (segment (start 88.4 69.9552) (end 87.4448 69) (width 0.25) (layer "F.Cu") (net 6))
 (via (at 88.4 70.5) (size 1) (drill 0.5) (layers "F.Cu" "B.Cu") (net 6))
 (segment (start 91.62 85.71) (end 79.87 97.46) (width 0.25) (layer "B.Cu") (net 6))
 (segment (start 90.55 70.5) (end 88.4 70.5) (width 0.25) (layer "B.Cu") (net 6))
 (segment (start 79.87 97.46) (end 79.87 96.44) (width 0.25) (layer "B.Cu") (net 6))
 (segment (start 91.62 71.57) (end 91.62 85.71) (width 0.25) (layer "B.Cu") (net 6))
 (segment (start 50.8 91.44) (end 61.59 91.44) (width 0.5) (layer "B.Cu") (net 6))
 (segment (start 91.62 71.57) (end 90.55 70.5) (width 0.25) (layer "B.Cu") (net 6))
 (segment (start 78.06 99.27) (end 79.87 97.46) (width 0.5) (layer "B.Cu") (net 6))
 (segment (start 61.59 91.44) (end 69.42 99.27) (width 0.5) (layer "B.Cu") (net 6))
 (segment (start 69.42 99.27) (end 78.06 99.27) (width 0.5) (layer "B.Cu") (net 6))
 (segment (start 53.49 93.98) (end 50.8 93.98) (width 2) (layer "F.Cu") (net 5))
 (segment (start 56.97 97.46) (end 53.49 93.98) (width 2) (layer "F.Cu") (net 5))
 (segment (start 88.7 60.93) (end 88.7 64.390278) (width 0.2) (layer "F.Cu") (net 20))
 (segment (start 88.7 64.390278) (end 84.6 68.490278) (width 0.2) (layer "F.Cu") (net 20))
 (segment (start 84.6 68.490278) (end 84.6 69) (width 0.2) (layer "F.Cu") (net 20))
 (segment (start 90.63 55.8) (end 90.63 59) (width 0.2) (layer "F.Cu") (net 20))
 (segment (start 90.63 59) (end 88.7 60.93) (width 0.2) (layer "F.Cu") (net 20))
 (segment (start 88.72 97.97) (end 88.72 97.370001) (width 0.5) (layer "F.Cu") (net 4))
 (segment (start 61.92 99.27) (end 87.42 99.27) (width 0.5) (layer "F.Cu") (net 4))
 (segment (start 54.8 75.5) (end 55.46 76.16) (width 0.5) (layer "F.Cu") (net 4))
 (segment (start 87.42 99.27) (end 88.72 97.97) (width 0.5) (layer "F.Cu") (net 4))
 (segment (start 88.72 97.370001) (end 91.52 94.570001) (width 0.5) (layer "F.Cu") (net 4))
 (segment (start 54.8 85.65) (end 54.8 75.5) (width 0.5) (layer "F.Cu") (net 4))
 (segment (start 50.8 88.9) (end 51.55 88.9) (width 0.5) (layer "F.Cu") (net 4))
 (segment (start 58.92 76.16) (end 58.92 96.27) (width 0.5) (layer "F.Cu") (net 4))
 (segment (start 51.55 88.9) (end 54.8 85.65) (width 0.5) (layer "F.Cu") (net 4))
 (segment (start 54.8 75.5) (end 58.7 71.6) (width 0.5) (layer "F.Cu") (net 4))
 (segment (start 61.92 99.27) (end 51.01 99.27) (width 0.5) (layer "F.Cu") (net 4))
 (segment (start 58.7 71.6) (end 87.8 71.6) (width 0.5) (layer "F.Cu") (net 4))
 (segment (start 58.92 96.27) (end 61.92 99.27) (width 0.5) (layer "F.Cu") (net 4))
 (segment (start 51.01 99.27) (end 50.8 99.06) (width 0.5) (layer "F.Cu") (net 4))
 (segment (start 55.46 76.16) (end 58.92 76.16) (width 0.5) (layer "F.Cu") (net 4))
 (via (at 87.8 71.6) (size 1.2) (drill 0.5) (layers "F.Cu" "B.Cu") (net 4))
 (segment (start 89.47 71.6) (end 90.6 72.73) (width 0.5) (layer "B.Cu") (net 4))
 (segment (start 87.8 71.6) (end 89.47 71.6) (width 0.5) (layer "B.Cu") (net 4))
 (segment (start 80.379997 62.7) (end 86.9 62.7) (width 1.5) (layer "F.Cu") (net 3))
 (segment (start 59.79 69.2) (end 56.6 69.2) (width 1.5) (layer "F.Cu") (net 3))
 (segment (start 52.512 82.278) (end 50.97 83.82) (width 1.5) (layer "F.Cu") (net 3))
 (segment (start 56.6 69.2) (end 52.512 73.288) (width 1.5) (layer "F.Cu") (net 3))
 (segment (start 77.919998 65.159999) (end 63.830001 65.159999) (width 1.5) (layer "F.Cu") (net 3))
 (segment (start 77.919998 65.159999) (end 80.379997 62.7) (width 1.5) (layer "F.Cu") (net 3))
 (segment (start 52.512 73.288) (end 52.512 82.278) (width 1.5) (layer "F.Cu") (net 3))
 (segment (start 63.830001 65.159999) (end 59.79 69.2) (width 1.5) (layer "F.Cu") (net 3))
 (segment (start 57.13 63.369999) (end 58.92 65.159999) (width 5) (layer "F.Cu") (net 21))
 (segment (start 57.13 60.15) (end 57.13 63.369999) (width 5) (layer "F.Cu") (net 21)))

